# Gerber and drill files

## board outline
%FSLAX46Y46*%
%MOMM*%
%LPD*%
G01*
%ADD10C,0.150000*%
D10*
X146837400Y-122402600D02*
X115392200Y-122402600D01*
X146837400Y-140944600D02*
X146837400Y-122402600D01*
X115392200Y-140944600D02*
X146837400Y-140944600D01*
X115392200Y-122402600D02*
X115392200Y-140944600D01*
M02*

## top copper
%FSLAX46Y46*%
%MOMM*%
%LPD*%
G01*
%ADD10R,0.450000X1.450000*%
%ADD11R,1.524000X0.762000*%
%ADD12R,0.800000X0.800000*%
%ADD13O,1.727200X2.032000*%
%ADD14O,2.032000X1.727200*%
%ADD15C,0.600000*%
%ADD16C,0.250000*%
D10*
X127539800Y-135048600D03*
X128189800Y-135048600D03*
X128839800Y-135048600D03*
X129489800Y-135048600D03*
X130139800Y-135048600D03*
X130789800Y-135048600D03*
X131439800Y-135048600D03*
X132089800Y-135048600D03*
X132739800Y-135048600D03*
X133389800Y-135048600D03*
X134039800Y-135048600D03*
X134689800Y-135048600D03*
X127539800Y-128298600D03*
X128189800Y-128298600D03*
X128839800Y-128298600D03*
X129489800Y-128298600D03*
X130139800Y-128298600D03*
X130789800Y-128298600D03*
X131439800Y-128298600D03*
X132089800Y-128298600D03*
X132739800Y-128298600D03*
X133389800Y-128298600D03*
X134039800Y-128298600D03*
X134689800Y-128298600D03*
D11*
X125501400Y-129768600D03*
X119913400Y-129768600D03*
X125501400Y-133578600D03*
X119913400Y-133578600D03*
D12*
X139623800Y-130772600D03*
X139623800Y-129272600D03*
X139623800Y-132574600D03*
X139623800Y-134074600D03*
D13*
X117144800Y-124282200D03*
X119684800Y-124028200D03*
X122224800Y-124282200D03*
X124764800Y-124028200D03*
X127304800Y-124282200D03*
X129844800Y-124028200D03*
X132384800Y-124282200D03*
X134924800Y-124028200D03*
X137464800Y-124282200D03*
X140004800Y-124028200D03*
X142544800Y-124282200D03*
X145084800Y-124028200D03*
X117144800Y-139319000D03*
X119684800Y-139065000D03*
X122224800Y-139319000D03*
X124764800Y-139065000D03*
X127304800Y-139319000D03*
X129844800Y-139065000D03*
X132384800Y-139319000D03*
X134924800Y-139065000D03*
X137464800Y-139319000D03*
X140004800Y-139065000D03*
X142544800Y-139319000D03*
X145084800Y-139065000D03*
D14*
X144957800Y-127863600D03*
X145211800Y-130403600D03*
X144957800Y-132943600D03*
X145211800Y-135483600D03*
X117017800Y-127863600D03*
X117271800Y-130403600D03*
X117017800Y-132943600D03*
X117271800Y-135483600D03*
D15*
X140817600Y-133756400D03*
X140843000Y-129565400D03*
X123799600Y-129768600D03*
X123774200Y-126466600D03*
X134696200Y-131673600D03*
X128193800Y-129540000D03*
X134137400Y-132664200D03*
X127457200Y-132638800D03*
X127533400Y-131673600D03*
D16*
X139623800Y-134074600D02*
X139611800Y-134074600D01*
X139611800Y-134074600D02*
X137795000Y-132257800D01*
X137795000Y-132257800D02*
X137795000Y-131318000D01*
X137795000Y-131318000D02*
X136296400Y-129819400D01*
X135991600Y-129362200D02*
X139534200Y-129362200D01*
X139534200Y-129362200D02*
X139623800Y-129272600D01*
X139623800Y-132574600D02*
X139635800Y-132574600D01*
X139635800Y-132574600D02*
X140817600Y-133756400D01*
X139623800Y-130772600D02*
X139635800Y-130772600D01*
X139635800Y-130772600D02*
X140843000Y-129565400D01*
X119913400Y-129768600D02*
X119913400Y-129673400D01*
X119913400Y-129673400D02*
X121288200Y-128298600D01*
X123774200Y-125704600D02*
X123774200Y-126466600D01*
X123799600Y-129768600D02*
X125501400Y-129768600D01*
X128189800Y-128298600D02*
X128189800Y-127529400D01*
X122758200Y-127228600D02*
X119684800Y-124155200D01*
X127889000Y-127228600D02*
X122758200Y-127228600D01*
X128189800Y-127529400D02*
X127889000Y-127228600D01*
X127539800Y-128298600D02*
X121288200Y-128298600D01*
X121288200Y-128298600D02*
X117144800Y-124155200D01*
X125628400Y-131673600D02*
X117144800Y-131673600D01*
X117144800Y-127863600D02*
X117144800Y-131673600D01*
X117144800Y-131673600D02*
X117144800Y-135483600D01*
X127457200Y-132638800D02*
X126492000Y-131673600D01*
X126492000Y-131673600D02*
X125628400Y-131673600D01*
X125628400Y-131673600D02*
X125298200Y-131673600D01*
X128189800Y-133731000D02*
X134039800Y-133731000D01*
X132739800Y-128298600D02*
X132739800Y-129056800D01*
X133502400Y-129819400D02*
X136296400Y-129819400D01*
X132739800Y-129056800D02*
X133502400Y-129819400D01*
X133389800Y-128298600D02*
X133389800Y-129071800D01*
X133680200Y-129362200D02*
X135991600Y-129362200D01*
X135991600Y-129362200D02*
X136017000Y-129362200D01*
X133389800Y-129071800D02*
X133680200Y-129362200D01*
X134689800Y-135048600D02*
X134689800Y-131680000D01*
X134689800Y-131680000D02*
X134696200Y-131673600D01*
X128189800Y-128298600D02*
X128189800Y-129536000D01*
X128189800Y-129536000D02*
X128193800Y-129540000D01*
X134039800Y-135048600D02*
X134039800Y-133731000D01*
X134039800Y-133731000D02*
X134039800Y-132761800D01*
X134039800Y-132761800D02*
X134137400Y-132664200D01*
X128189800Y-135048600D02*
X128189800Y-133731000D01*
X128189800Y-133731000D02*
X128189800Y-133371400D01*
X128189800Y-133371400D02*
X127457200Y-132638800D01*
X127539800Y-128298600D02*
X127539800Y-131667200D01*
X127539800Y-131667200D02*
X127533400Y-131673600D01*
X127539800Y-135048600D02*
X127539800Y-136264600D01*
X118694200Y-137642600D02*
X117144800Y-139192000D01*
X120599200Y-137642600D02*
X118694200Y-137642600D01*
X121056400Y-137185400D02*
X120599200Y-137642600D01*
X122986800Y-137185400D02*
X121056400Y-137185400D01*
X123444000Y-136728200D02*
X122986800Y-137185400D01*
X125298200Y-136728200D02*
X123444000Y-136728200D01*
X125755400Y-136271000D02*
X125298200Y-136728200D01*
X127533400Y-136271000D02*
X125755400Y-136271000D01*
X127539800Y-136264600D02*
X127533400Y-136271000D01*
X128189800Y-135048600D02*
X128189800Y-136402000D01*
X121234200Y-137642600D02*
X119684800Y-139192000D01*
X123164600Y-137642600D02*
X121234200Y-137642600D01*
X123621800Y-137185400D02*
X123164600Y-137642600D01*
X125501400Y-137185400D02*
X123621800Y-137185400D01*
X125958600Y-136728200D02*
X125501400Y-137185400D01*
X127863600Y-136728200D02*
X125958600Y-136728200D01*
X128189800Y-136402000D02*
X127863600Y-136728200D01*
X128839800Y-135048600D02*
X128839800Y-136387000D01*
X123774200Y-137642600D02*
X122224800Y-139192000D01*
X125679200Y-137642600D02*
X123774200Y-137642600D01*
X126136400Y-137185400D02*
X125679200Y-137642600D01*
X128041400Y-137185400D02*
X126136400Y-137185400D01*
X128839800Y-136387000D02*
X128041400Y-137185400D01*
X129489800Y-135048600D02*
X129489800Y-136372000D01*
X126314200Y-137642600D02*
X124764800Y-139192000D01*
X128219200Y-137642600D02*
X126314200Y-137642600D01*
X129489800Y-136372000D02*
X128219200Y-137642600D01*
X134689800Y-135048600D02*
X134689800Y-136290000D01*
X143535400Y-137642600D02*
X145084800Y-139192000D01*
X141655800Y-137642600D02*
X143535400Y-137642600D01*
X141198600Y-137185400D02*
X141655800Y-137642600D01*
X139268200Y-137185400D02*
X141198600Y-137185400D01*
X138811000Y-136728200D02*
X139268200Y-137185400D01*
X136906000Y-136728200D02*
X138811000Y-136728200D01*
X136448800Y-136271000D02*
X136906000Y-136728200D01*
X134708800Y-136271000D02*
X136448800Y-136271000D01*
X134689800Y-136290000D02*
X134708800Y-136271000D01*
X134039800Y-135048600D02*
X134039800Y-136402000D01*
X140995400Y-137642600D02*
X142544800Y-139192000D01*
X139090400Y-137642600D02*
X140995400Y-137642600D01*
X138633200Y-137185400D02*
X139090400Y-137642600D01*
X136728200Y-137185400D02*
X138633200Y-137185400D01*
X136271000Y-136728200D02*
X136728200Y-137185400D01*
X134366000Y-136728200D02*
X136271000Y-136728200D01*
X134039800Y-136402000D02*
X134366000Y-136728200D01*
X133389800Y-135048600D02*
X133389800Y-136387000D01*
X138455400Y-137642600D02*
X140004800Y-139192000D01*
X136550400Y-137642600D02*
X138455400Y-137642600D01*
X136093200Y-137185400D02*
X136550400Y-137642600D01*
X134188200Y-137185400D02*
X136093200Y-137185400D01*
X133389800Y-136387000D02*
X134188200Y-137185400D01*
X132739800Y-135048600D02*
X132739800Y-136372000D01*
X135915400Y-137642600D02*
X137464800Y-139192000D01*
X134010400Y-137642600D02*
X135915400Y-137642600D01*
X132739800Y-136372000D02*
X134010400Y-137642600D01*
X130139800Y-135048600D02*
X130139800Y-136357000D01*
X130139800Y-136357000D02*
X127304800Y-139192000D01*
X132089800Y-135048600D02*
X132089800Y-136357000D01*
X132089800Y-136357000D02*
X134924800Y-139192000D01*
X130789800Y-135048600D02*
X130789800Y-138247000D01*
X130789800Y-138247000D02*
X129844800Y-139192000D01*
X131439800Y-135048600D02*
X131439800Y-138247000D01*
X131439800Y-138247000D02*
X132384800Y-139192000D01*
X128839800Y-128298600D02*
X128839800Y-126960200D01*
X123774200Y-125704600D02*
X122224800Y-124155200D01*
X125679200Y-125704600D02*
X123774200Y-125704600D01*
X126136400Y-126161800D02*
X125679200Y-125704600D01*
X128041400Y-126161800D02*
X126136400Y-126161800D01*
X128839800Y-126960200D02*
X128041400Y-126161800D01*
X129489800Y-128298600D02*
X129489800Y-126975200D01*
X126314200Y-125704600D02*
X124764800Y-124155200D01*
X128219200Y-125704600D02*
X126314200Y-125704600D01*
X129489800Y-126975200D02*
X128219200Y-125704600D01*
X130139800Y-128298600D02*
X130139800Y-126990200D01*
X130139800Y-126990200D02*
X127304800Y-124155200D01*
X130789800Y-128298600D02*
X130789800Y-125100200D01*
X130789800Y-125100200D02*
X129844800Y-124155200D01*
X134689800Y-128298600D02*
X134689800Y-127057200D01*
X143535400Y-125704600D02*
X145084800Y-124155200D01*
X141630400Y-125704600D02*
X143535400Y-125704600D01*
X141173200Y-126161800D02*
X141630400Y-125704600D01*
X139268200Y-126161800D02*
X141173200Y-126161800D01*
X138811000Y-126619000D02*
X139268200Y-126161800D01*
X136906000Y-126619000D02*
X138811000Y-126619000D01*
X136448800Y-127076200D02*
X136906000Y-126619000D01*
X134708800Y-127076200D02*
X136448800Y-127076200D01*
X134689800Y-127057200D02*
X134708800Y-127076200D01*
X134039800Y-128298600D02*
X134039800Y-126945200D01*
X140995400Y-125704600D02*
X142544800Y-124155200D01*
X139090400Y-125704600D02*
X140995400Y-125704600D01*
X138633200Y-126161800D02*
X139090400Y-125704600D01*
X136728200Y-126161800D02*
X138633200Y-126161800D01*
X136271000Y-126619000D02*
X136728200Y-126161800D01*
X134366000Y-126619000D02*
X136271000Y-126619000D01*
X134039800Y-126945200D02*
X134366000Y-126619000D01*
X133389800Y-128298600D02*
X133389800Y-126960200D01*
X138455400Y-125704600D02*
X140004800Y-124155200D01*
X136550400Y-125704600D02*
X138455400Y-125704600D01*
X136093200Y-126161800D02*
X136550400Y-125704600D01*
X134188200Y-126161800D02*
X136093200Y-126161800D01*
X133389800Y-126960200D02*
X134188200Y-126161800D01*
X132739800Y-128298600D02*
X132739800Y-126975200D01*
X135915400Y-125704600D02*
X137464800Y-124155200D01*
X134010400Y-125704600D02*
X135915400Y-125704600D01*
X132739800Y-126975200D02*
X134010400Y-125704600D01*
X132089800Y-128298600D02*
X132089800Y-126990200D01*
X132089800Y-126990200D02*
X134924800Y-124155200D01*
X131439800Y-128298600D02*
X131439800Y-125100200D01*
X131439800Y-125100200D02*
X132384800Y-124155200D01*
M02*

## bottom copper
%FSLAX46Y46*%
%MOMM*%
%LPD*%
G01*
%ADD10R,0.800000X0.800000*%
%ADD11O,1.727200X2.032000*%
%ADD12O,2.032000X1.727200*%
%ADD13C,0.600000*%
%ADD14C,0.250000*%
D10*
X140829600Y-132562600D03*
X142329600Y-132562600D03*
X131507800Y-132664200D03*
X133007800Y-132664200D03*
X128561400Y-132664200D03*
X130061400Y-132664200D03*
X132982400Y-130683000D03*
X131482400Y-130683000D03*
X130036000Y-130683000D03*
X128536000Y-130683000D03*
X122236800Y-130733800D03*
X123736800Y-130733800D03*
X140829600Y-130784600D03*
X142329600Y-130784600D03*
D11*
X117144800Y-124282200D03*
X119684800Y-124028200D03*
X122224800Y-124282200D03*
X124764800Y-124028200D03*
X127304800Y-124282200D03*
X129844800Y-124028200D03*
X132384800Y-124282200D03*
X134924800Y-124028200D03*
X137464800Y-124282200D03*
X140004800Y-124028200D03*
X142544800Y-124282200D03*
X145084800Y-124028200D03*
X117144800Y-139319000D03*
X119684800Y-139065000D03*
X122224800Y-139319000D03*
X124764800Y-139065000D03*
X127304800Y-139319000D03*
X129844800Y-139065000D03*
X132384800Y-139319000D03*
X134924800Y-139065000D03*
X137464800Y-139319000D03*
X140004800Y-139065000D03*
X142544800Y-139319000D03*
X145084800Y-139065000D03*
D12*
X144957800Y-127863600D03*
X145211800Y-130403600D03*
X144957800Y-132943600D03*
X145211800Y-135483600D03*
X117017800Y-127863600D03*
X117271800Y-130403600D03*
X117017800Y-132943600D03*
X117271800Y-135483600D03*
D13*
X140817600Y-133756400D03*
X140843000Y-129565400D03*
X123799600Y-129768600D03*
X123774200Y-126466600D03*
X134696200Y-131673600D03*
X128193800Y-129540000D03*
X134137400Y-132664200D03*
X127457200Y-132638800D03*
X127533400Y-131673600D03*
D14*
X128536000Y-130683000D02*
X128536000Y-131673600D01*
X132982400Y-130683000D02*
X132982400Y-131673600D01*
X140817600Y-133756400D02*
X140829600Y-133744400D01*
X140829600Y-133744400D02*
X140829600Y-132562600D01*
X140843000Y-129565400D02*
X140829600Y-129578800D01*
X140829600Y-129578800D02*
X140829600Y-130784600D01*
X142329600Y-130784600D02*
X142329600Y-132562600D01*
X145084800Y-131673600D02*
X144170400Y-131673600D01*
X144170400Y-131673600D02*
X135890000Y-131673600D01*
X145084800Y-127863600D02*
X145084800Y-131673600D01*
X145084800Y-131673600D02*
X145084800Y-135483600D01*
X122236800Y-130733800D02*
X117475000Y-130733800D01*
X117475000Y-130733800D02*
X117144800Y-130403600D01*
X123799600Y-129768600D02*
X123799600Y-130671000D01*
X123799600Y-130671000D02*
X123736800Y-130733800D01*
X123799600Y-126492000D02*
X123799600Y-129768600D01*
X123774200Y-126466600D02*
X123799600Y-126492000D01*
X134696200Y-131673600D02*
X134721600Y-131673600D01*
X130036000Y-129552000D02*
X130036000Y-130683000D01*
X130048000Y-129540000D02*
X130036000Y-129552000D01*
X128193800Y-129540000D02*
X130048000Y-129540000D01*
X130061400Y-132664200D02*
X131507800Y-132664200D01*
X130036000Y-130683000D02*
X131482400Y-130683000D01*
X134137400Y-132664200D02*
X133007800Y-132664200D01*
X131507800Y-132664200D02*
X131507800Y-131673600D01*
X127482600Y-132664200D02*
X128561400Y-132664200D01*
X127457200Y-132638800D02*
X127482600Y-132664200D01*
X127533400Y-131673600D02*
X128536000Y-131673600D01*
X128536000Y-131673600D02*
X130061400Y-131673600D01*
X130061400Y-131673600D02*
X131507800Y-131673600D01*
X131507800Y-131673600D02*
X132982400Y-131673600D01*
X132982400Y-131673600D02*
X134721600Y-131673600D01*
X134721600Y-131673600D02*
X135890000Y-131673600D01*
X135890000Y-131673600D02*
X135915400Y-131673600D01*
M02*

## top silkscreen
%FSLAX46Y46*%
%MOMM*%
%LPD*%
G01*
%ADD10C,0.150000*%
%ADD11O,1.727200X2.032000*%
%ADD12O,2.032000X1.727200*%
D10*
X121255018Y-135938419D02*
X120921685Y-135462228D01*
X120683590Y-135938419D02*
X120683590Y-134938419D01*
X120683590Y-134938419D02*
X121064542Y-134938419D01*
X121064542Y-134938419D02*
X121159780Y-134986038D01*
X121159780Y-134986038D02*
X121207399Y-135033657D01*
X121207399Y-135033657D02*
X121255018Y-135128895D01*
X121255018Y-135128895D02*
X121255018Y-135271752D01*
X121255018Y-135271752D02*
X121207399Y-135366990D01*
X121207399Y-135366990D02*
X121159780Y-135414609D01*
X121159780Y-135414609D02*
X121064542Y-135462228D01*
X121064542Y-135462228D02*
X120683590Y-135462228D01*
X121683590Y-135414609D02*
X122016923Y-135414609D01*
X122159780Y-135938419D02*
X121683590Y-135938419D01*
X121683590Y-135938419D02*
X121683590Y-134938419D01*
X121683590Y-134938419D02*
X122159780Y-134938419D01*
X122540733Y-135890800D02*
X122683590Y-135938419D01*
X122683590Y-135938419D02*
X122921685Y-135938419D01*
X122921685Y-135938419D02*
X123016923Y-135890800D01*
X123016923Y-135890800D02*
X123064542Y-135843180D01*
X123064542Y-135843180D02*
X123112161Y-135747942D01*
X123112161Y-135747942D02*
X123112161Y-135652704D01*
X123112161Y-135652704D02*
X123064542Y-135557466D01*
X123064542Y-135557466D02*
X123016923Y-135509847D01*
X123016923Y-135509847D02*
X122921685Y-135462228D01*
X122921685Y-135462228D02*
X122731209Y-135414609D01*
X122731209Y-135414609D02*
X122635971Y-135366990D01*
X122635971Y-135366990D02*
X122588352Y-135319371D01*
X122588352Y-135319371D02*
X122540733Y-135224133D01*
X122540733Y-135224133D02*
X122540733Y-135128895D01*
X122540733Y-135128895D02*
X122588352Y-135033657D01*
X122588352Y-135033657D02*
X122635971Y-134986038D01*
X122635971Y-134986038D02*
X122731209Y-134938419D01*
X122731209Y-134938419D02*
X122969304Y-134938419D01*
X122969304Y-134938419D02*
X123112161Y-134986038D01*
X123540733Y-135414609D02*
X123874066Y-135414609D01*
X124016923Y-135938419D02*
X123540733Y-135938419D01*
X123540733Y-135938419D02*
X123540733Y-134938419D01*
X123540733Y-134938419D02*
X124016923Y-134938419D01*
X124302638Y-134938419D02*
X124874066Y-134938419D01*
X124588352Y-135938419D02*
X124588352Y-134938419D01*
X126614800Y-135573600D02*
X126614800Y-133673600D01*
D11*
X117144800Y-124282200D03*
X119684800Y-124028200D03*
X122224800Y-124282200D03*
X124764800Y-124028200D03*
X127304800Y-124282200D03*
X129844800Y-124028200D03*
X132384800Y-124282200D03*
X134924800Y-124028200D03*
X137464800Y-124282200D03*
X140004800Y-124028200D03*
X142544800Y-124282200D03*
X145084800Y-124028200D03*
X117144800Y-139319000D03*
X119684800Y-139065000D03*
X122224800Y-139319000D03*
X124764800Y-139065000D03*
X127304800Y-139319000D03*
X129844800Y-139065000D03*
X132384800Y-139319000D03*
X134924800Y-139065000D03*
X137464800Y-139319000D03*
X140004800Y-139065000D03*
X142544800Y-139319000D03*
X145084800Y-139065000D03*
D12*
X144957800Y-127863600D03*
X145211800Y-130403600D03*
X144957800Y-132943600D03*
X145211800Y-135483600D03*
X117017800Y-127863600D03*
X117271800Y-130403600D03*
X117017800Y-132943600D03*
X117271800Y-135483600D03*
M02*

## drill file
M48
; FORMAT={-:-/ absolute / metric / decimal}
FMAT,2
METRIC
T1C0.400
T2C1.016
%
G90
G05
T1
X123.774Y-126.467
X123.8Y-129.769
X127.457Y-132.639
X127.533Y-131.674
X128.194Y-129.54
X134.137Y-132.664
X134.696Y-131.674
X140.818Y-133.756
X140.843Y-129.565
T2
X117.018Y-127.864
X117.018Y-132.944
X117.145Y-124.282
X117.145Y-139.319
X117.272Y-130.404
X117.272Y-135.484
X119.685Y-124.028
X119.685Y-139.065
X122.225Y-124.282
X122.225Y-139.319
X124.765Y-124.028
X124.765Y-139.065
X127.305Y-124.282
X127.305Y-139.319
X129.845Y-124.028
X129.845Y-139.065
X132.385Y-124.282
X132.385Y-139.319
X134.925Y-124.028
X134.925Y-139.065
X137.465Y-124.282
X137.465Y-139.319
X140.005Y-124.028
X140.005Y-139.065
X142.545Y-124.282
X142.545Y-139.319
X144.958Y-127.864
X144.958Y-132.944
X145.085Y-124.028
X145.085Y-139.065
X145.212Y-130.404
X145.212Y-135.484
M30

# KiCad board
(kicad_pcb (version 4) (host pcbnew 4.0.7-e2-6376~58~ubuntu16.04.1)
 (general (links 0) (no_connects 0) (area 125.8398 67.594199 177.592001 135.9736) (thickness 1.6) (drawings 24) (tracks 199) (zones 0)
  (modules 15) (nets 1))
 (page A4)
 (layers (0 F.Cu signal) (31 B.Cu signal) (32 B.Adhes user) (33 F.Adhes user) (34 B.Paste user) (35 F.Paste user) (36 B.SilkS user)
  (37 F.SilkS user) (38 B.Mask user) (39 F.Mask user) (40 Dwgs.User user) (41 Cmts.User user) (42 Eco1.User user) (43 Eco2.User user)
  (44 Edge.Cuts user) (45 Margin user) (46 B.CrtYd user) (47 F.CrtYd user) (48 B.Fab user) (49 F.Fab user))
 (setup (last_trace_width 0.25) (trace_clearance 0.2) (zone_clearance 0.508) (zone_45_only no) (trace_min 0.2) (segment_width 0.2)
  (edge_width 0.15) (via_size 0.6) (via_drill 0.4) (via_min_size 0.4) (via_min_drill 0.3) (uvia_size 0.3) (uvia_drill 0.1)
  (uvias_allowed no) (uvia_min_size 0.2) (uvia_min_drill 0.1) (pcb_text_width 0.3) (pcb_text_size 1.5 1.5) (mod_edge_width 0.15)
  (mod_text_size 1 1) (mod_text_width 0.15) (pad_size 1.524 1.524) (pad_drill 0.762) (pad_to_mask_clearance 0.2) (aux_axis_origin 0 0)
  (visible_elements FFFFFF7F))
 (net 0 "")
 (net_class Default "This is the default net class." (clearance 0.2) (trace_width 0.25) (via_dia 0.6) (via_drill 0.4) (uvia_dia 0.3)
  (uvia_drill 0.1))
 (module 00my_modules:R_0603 (layer B.Cu) (at 141.5796 132.5626)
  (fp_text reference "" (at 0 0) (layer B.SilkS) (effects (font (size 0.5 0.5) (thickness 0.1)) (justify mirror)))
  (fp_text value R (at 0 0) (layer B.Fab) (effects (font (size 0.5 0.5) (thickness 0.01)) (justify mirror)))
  (pad 1 smd rect (at -0.75 0) (size 0.8 0.8) (layers B.Cu B.Paste B.Mask))
  (pad 2 smd rect (at 0.75 0) (size 0.8 0.8) (layers B.Cu B.Paste B.Mask)))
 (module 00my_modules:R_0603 (layer B.Cu) (at 132.2578 132.6642)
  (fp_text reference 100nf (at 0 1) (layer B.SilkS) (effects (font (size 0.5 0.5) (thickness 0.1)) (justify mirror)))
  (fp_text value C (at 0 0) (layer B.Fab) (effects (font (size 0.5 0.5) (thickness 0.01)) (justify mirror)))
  (pad 1 smd rect (at -0.75 0) (size 0.8 0.8) (layers B.Cu B.Paste B.Mask))
  (pad 2 smd rect (at 0.75 0) (size 0.8 0.8) (layers B.Cu B.Paste B.Mask)))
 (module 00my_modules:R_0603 (layer B.Cu) (at 129.3114 132.6642)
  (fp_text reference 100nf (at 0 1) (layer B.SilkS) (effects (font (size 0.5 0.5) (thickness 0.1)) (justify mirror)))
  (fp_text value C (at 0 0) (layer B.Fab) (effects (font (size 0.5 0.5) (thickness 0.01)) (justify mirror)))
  (pad 1 smd rect (at -0.75 0) (size 0.8 0.8) (layers B.Cu B.Paste B.Mask))
  (pad 2 smd rect (at 0.75 0) (size 0.8 0.8) (layers B.Cu B.Paste B.Mask)))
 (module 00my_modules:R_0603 (layer B.Cu) (at 132.2324 130.683 180)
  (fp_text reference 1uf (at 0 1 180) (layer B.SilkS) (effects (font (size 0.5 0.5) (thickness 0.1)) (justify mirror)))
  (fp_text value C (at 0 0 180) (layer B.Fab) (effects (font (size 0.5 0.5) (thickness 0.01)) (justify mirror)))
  (pad 1 smd rect (at -0.75 0 180) (size 0.8 0.8) (layers B.Cu B.Paste B.Mask))
  (pad 2 smd rect (at 0.75 0 180) (size 0.8 0.8) (layers B.Cu B.Paste B.Mask)))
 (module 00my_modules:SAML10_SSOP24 (layer F.Cu) (at 131.1148 131.6736 90)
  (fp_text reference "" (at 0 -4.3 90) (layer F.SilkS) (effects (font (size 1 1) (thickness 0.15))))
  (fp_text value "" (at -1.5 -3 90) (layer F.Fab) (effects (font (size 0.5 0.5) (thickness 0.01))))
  (fp_line (start -3.9 -4.5) (end -2 -4.5) (layer F.SilkS) (width 0.15))
  (pad VOUT smd rect (at -3.375 -3.575 90) (size 1.45 0.45) (layers F.Cu F.Paste F.Mask))
  (pad VIO smd rect (at -3.375 -2.925 90) (size 1.45 0.45) (layers F.Cu F.Paste F.Mask))
  (pad SWCL smd rect (at -3.375 -2.275 90) (size 1.45 0.45) (layers F.Cu F.Paste F.Mask))
  (pad SWDI smd rect (at -3.375 -1.625 90) (size 1.45 0.45) (layers F.Cu F.Paste F.Mask))
  (pad PA00 smd rect (at -3.375 -0.975 90) (size 1.45 0.45) (layers F.Cu F.Paste F.Mask))
  (pad PA01 smd rect (at -3.375 -0.325 90) (size 1.45 0.45) (layers F.Cu F.Paste F.Mask))
  (pad PA02 smd rect (at -3.375 0.325 90) (size 1.45 0.45) (layers F.Cu F.Paste F.Mask))
  (pad PA03 smd rect (at -3.375 0.975 90) (size 1.45 0.45) (layers F.Cu F.Paste F.Mask))
  (pad PA04 smd rect (at -3.375 1.625 90) (size 1.45 0.45) (layers F.Cu F.Paste F.Mask))
  (pad PA05 smd rect (at -3.375 2.275 90) (size 1.45 0.45) (layers F.Cu F.Paste F.Mask))
  (pad VANA smd rect (at -3.375 2.925 90) (size 1.45 0.45) (layers F.Cu F.Paste F.Mask))
  (pad GANA smd rect (at -3.375 3.575 90) (size 1.45 0.45) (layers F.Cu F.Paste F.Mask))
  (pad GND smd rect (at 3.375 -3.575 90) (size 1.45 0.45) (layers F.Cu F.Paste F.Mask))
  (pad VCOR smd rect (at 3.375 -2.925 90) (size 1.45 0.45) (layers F.Cu F.Paste F.Mask))
  (pad RSTN smd rect (at 3.375 -2.275 90) (size 1.45 0.45) (layers F.Cu F.Paste F.Mask))
  (pad PA23 smd rect (at 3.375 -1.625 90) (size 1.45 0.45) (layers F.Cu F.Paste F.Mask))
  (pad PA22 smd rect (at 3.375 -0.975 90) (size 1.45 0.45) (layers F.Cu F.Paste F.Mask))
  (pad PA19 smd rect (at 3.375 -0.325 90) (size 1.45 0.45) (layers F.Cu F.Paste F.Mask))
  (pad PA18 smd rect (at 3.375 0.325 90) (size 1.45 0.45) (layers F.Cu F.Paste F.Mask))
  (pad PA17 smd rect (at 3.375 0.975 90) (size 1.45 0.45) (layers F.Cu F.Paste F.Mask))
  (pad PA16 smd rect (at 3.375 1.625 90) (size 1.45 0.45) (layers F.Cu F.Paste F.Mask))
  (pad PA15 smd rect (at 3.375 2.275 90) (size 1.45 0.45) (layers F.Cu F.Paste F.Mask))
  (pad PA14 smd rect (at 3.375 2.925 90) (size 1.45 0.45) (layers F.Cu F.Paste F.Mask))
  (pad PA08 smd rect (at 3.375 3.575 90) (size 1.45 0.45) (layers F.Cu F.Paste F.Mask)))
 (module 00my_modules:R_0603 (layer B.Cu) (at 129.286 130.683 180)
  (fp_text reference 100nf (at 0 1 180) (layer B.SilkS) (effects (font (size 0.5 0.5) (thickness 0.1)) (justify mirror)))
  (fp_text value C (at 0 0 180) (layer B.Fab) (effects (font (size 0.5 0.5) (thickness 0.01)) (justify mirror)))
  (pad 1 smd rect (at -0.75 0 180) (size 0.8 0.8) (layers B.Cu B.Paste B.Mask))
  (pad 2 smd rect (at 0.75 0 180) (size 0.8 0.8) (layers B.Cu B.Paste B.Mask)))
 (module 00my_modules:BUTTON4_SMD (layer F.Cu) (at 122.7074 131.6736 180)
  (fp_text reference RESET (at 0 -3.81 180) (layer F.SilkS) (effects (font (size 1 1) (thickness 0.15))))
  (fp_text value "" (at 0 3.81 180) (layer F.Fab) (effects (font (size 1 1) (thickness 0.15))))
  (pad 1 smd rect (at -2.794 1.905 180) (size 1.524 0.762) (layers F.Cu F.Paste F.Mask))
  (pad 2 smd rect (at 2.794 1.905 180) (size 1.524 0.762) (layers F.Cu F.Paste F.Mask))
  (pad 3 smd rect (at -2.794 -1.905 180) (size 1.524 0.762) (layers F.Cu F.Paste F.Mask))
  (pad 4 smd rect (at 2.794 -1.905 180) (size 1.524 0.762) (layers F.Cu F.Paste F.Mask)))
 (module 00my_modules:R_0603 (layer B.Cu) (at 122.9868 130.7338)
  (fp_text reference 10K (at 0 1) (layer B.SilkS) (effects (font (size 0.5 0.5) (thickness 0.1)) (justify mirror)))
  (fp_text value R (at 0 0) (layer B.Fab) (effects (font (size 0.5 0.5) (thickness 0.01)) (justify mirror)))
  (pad 1 smd rect (at -0.75 0) (size 0.8 0.8) (layers B.Cu B.Paste B.Mask))
  (pad 2 smd rect (at 0.75 0) (size 0.8 0.8) (layers B.Cu B.Paste B.Mask)))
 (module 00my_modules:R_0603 (layer B.Cu) (at 141.5796 130.7846)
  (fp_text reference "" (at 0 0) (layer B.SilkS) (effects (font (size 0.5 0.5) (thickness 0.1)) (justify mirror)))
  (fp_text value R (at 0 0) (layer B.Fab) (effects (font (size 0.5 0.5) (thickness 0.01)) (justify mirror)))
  (pad 1 smd rect (at -0.75 0) (size 0.8 0.8) (layers B.Cu B.Paste B.Mask))
  (pad 2 smd rect (at 0.75 0) (size 0.8 0.8) (layers B.Cu B.Paste B.Mask)))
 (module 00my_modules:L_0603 (layer F.Cu) (at 139.6238 130.0226 90)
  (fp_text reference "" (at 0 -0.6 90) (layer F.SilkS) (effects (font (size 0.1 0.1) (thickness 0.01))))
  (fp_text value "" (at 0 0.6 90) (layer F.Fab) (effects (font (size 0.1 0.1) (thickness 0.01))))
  (pad 1 smd rect (at -0.75 0 90) (size 0.8 0.8) (layers F.Cu F.Paste F.Mask))
  (pad 2 smd rect (at 0.75 0 90) (size 0.8 0.8) (layers F.Cu F.Paste F.Mask)))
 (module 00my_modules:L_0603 (layer F.Cu) (at 139.6238 133.3246 270)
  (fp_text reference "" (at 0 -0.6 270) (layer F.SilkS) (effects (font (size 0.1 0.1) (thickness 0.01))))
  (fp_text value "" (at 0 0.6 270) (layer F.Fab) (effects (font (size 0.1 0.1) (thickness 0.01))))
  (pad 1 smd rect (at -0.75 0 270) (size 0.8 0.8) (layers F.Cu F.Paste F.Mask))
  (pad 2 smd rect (at 0.75 0 270) (size 0.8 0.8) (layers F.Cu F.Paste F.Mask)))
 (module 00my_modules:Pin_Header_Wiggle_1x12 (layer F.Cu) (at 117.1448 124.1552 90)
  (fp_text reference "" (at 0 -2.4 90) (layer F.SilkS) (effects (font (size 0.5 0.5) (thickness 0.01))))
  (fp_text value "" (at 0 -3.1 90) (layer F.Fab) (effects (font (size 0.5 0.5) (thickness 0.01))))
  (pad 1 thru_hole oval (at -0.127 0 90) (size 2.032 1.7272) (drill 1.016) (layers *.Cu *.Mask F.SilkS))
  (pad 2 thru_hole oval (at 0.127 2.54 90) (size 2.032 1.7272) (drill 1.016) (layers *.Cu *.Mask F.SilkS))
  (pad 3 thru_hole oval (at -0.127 5.08 90) (size 2.032 1.7272) (drill 1.016) (layers *.Cu *.Mask F.SilkS))
  (pad 4 thru_hole oval (at 0.127 7.62 90) (size 2.032 1.7272) (drill 1.016) (layers *.Cu *.Mask F.SilkS))
  (pad 5 thru_hole oval (at -0.127 10.16 90) (size 2.032 1.7272) (drill 1.016) (layers *.Cu *.Mask F.SilkS))
  (pad 6 thru_hole oval (at 0.127 12.7 90) (size 2.032 1.7272) (drill 1.016) (layers *.Cu *.Mask F.SilkS))
  (pad 7 thru_hole oval (at -0.127 15.24 90) (size 2.032 1.7272) (drill 1.016) (layers *.Cu *.Mask F.SilkS))
  (pad 8 thru_hole oval (at 0.127 17.78 90) (size 2.032 1.7272) (drill 1.016) (layers *.Cu *.Mask F.SilkS))
  (pad 9 thru_hole oval (at -0.127 20.32 90) (size 2.032 1.7272) (drill 1.016) (layers *.Cu *.Mask F.SilkS))
  (pad 10 thru_hole oval (at 0.127 22.86 90) (size 2.032 1.7272) (drill 1.016) (layers *.Cu *.Mask F.SilkS))
  (pad 11 thru_hole oval (at -0.127 25.4 90) (size 2.032 1.7272) (drill 1.016) (layers *.Cu *.Mask F.SilkS))
  (pad 12 thru_hole oval (at 0.127 27.94 90) (size 2.032 1.7272) (drill 1.016) (layers *.Cu *.Mask F.SilkS)))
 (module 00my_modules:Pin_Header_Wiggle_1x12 (layer F.Cu) (at 117.1448 139.192 90)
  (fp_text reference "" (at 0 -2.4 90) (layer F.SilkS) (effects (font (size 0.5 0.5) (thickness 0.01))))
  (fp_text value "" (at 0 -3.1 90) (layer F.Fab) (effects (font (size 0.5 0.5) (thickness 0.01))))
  (pad 1 thru_hole oval (at -0.127 0 90) (size 2.032 1.7272) (drill 1.016) (layers *.Cu *.Mask F.SilkS))
  (pad 2 thru_hole oval (at 0.127 2.54 90) (size 2.032 1.7272) (drill 1.016) (layers *.Cu *.Mask F.SilkS))
  (pad 3 thru_hole oval (at -0.127 5.08 90) (size 2.032 1.7272) (drill 1.016) (layers *.Cu *.Mask F.SilkS))
  (pad 4 thru_hole oval (at 0.127 7.62 90) (size 2.032 1.7272) (drill 1.016) (layers *.Cu *.Mask F.SilkS))
  (pad 5 thru_hole oval (at -0.127 10.16 90) (size 2.032 1.7272) (drill 1.016) (layers *.Cu *.Mask F.SilkS))
  (pad 6 thru_hole oval (at 0.127 12.7 90) (size 2.032 1.7272) (drill 1.016) (layers *.Cu *.Mask F.SilkS))
  (pad 7 thru_hole oval (at -0.127 15.24 90) (size 2.032 1.7272) (drill 1.016) (layers *.Cu *.Mask F.SilkS))
  (pad 8 thru_hole oval (at 0.127 17.78 90) (size 2.032 1.7272) (drill 1.016) (layers *.Cu *.Mask F.SilkS))
  (pad 9 thru_hole oval (at -0.127 20.32 90) (size 2.032 1.7272) (drill 1.016) (layers *.Cu *.Mask F.SilkS))
  (pad 10 thru_hole oval (at 0.127 22.86 90) (size 2.032 1.7272) (drill 1.016) (layers *.Cu *.Mask F.SilkS))
  (pad 11 thru_hole oval (at -0.127 25.4 90) (size 2.032 1.7272) (drill 1.016) (layers *.Cu *.Mask F.SilkS))
  (pad 12 thru_hole oval (at 0.127 27.94 90) (size 2.032 1.7272) (drill 1.016) (layers *.Cu *.Mask F.SilkS)))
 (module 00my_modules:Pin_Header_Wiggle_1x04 (layer F.Cu) (at 145.0848 127.8636)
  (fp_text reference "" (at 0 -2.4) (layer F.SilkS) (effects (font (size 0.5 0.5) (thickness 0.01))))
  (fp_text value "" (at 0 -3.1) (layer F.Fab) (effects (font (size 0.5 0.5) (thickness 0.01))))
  (pad 1 thru_hole oval (at -0.127 0) (size 2.032 1.7272) (drill 1.016) (layers *.Cu *.Mask F.SilkS))
  (pad 2 thru_hole oval (at 0.127 2.54) (size 2.032 1.7272) (drill 1.016) (layers *.Cu *.Mask F.SilkS))
  (pad 3 thru_hole oval (at -0.127 5.08) (size 2.032 1.7272) (drill 1.016) (layers *.Cu *.Mask F.SilkS))
  (pad 4 thru_hole oval (at 0.127 7.62) (size 2.032 1.7272) (drill 1.016) (layers *.Cu *.Mask F.SilkS)))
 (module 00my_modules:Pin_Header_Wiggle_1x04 (layer F.Cu) (at 117.1448 127.8636)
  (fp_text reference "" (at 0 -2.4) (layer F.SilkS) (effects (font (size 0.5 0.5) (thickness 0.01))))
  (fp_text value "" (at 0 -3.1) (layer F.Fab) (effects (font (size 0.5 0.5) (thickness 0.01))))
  (pad 1 thru_hole oval (at -0.127 0) (size 2.032 1.7272) (drill 1.016) (layers *.Cu *.Mask F.SilkS))
  (pad 2 thru_hole oval (at 0.127 2.54) (size 2.032 1.7272) (drill 1.016) (layers *.Cu *.Mask F.SilkS))
  (pad 3 thru_hole oval (at -0.127 5.08) (size 2.032 1.7272) (drill 1.016) (layers *.Cu *.Mask F.SilkS))
  (pad 4 thru_hole oval (at 0.127 7.62) (size 2.032 1.7272) (drill 1.016) (layers *.Cu *.Mask F.SilkS)))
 (gr_line (start 146.8374 122.4026) (end 115.3922 122.4026) (angle 90) (layer Edge.Cuts) (width 0.15))
 (gr_line (start 146.8374 140.9446) (end 146.8374 122.4026) (angle 90) (layer Edge.Cuts) (width 0.15))
 (gr_line (start 115.3922 140.9446) (end 146.8374 140.9446) (angle 90) (layer Edge.Cuts) (width 0.15))
 (gr_line (start 115.3922 122.4026) (end 115.3922 140.9446) (angle 90) (layer Edge.Cuts) (width 0.15))
 (segment (start 128.536 130.683) (end 128.536 131.6736) (width 0.25) (layer B.Cu) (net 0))
 (segment (start 132.9824 130.683) (end 132.9824 131.6736) (width 0.25) (layer B.Cu) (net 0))
 (segment (start 139.6238 134.0746) (end 139.6118 134.0746) (width 0.25) (layer F.Cu) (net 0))
 (segment (start 139.6118 134.0746) (end 137.795 132.2578) (width 0.25) (layer F.Cu) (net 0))
 (segment (start 137.795 132.2578) (end 137.795 131.318) (width 0.25) (layer F.Cu) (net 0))
 (segment (start 137.795 131.318) (end 136.2964 129.8194) (width 0.25) (layer F.Cu) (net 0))
 (segment (start 135.9916 129.3622) (end 139.5342 129.3622) (width 0.25) (layer F.Cu) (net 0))
 (segment (start 139.5342 129.3622) (end 139.6238 129.2726) (width 0.25) (layer F.Cu) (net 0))
 (segment (start 139.6238 132.5746) (end 139.6358 132.5746) (width 0.25) (layer F.Cu) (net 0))
 (segment (start 139.6358 132.5746) (end 140.8176 133.7564) (width 0.25) (layer F.Cu) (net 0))
 (via (at 140.8176 133.7564) (size 0.6) (drill 0.4) (layers F.Cu B.Cu) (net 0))
 (segment (start 140.8176 133.7564) (end 140.8296 133.7444) (width 0.25) (layer B.Cu) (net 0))
 (segment (start 140.8296 133.7444) (end 140.8296 132.5626) (width 0.25) (layer B.Cu) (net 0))
 (segment (start 139.6238 130.7726) (end 139.6358 130.7726) (width 0.25) (layer F.Cu) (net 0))
 (segment (start 139.6358 130.7726) (end 140.843 129.5654) (width 0.25) (layer F.Cu) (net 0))
 (via (at 140.843 129.5654) (size 0.6) (drill 0.4) (layers F.Cu B.Cu) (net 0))
 (segment (start 140.843 129.5654) (end 140.8296 129.5788) (width 0.25) (layer B.Cu) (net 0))
 (segment (start 140.8296 129.5788) (end 140.8296 130.7846) (width 0.25) (layer B.Cu) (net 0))
 (segment (start 142.3296 130.7846) (end 142.3296 132.5626) (width 0.25) (layer B.Cu) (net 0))
 (segment (start 145.0848 131.6736) (end 144.1704 131.6736) (width 0.25) (layer B.Cu) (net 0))
 (segment (start 144.1704 131.6736) (end 135.89 131.6736) (width 0.25) (layer B.Cu) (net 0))
 (segment (start 145.0848 127.8636) (end 145.0848 131.6736) (width 0.25) (layer B.Cu) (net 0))
 (segment (start 145.0848 131.6736) (end 145.0848 135.4836) (width 0.25) (layer B.Cu) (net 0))
 (segment (start 122.2368 130.7338) (end 117.475 130.7338) (width 0.25) (layer B.Cu) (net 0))
 (segment (start 117.475 130.7338) (end 117.1448 130.4036) (width 0.25) (layer B.Cu) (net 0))
 (segment (start 123.7996 129.7686) (end 123.7996 130.671) (width 0.25) (layer B.Cu) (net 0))
 (segment (start 123.7996 130.671) (end 123.7368 130.7338) (width 0.25) (layer B.Cu) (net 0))
 (segment (start 119.9134 129.7686) (end 119.9134 129.6734) (width 0.25) (layer F.Cu) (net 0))
 (segment (start 119.9134 129.6734) (end 121.2882 128.2986) (width 0.25) (layer F.Cu) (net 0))
 (segment (start 123.7742 125.7046) (end 123.7742 126.4666) (width 0.25) (layer F.Cu) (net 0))
 (segment (start 123.7996 129.7686) (end 125.5014 129.7686) (width 0.25) (layer F.Cu) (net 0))
 (via (at 123.7996 129.7686) (size 0.6) (drill 0.4) (layers F.Cu B.Cu) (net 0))
 (segment (start 123.7996 126.492) (end 123.7996 129.7686) (width 0.25) (layer B.Cu) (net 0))
 (segment (start 123.7742 126.4666) (end 123.7996 126.492) (width 0.25) (layer B.Cu) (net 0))
 (via (at 123.7742 126.4666) (size 0.6) (drill 0.4) (layers F.Cu B.Cu) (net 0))
 (segment (start 128.1898 128.2986) (end 128.1898 127.5294) (width 0.25) (layer F.Cu) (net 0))
 (segment (start 122.7582 127.2286) (end 119.6848 124.1552) (width 0.25) (layer F.Cu) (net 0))
 (segment (start 127.889 127.2286) (end 122.7582 127.2286) (width 0.25) (layer F.Cu) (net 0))
 (segment (start 128.1898 127.5294) (end 127.889 127.2286) (width 0.25) (layer F.Cu) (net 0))
 (segment (start 127.5398 128.2986) (end 121.2882 128.2986) (width 0.25) (layer F.Cu) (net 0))
 (segment (start 121.2882 128.2986) (end 117.1448 124.1552) (width 0.25) (layer F.Cu) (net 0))
 (segment (start 125.6284 131.6736) (end 117.1448 131.6736) (width 0.25) (layer F.Cu) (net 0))
 (segment (start 117.1448 127.8636) (end 117.1448 131.6736) (width 0.25) (layer F.Cu) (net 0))
 (segment (start 117.1448 131.6736) (end 117.1448 135.4836) (width 0.25) (layer F.Cu) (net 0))
 (segment (start 127.4572 132.6388) (end 126.492 131.6736) (width 0.25) (layer F.Cu) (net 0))
 (segment (start 126.492 131.6736) (end 125.6284 131.6736) (width 0.25) (layer F.Cu) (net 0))
 (segment (start 125.6284 131.6736) (end 125.2982 131.6736) (width 0.25) (layer F.Cu) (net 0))
 (segment (start 128.1898 133.731) (end 134.0398 133.731) (width 0.25) (layer F.Cu) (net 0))
 (segment (start 132.7398 128.2986) (end 132.7398 129.0568) (width 0.25) (layer F.Cu) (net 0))
 (segment (start 133.5024 129.8194) (end 136.2964 129.8194) (width 0.25) (layer F.Cu) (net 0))
 (segment (start 132.7398 129.0568) (end 133.5024 129.8194) (width 0.25) (layer F.Cu) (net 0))
 (segment (start 133.3898 128.2986) (end 133.3898 129.0718) (width 0.25) (layer F.Cu) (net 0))
 (segment (start 133.6802 129.3622) (end 135.9916 129.3622) (width 0.25) (layer F.Cu) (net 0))
 (segment (start 135.9916 129.3622) (end 136.017 129.3622) (width 0.25) (layer F.Cu) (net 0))
 (segment (start 133.3898 129.0718) (end 133.6802 129.3622) (width 0.25) (layer F.Cu) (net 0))
 (segment (start 134.6898 135.0486) (end 134.6898 131.68) (width 0.25) (layer F.Cu) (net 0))
 (segment (start 134.6962 131.6736) (end 134.7216 131.6736) (width 0.25) (layer B.Cu) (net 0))
 (via (at 134.6962 131.6736) (size 0.6) (drill 0.4) (layers F.Cu B.Cu) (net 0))
 (segment (start 134.6898 131.68) (end 134.6962 131.6736) (width 0.25) (layer F.Cu) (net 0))
 (segment (start 128.1898 128.2986) (end 128.1898 129.536) (width 0.25) (layer F.Cu) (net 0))
 (segment (start 130.036 129.552) (end 130.036 130.683) (width 0.25) (layer B.Cu) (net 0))
 (segment (start 130.048 129.54) (end 130.036 129.552) (width 0.25) (layer B.Cu) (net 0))
 (segment (start 128.1938 129.54) (end 130.048 129.54) (width 0.25) (layer B.Cu) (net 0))
 (via (at 128.1938 129.54) (size 0.6) (drill 0.4) (layers F.Cu B.Cu) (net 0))
 (segment (start 128.1898 129.536) (end 128.1938 129.54) (width 0.25) (layer F.Cu) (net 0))
 (segment (start 130.0614 132.6642) (end 131.5078 132.6642) (width 0.25) (layer B.Cu) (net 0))
 (segment (start 130.036 130.683) (end 131.4824 130.683) (width 0.25) (layer B.Cu) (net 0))
 (segment (start 134.0398 135.0486) (end 134.0398 133.731) (width 0.25) (layer F.Cu) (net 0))
 (segment (start 134.0398 133.731) (end 134.0398 132.7618) (width 0.25) (layer F.Cu) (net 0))
 (segment (start 134.0398 132.7618) (end 134.1374 132.6642) (width 0.25) (layer F.Cu) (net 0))
 (via (at 134.1374 132.6642) (size 0.6) (drill 0.4) (layers F.Cu B.Cu) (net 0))
 (segment (start 134.1374 132.6642) (end 133.0078 132.6642) (width 0.25) (layer B.Cu) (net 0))
 (segment (start 131.5078 132.6642) (end 131.5078 131.6736) (width 0.25) (layer B.Cu) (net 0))
 (segment (start 128.1898 135.0486) (end 128.1898 133.731) (width 0.25) (layer F.Cu) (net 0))
 (segment (start 128.1898 133.731) (end 128.1898 133.3714) (width 0.25) (layer F.Cu) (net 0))
 (segment (start 127.4826 132.6642) (end 128.5614 132.6642) (width 0.25) (layer B.Cu) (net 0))
 (segment (start 127.4572 132.6388) (end 127.4826 132.6642) (width 0.25) (layer B.Cu) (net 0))
 (via (at 127.4572 132.6388) (size 0.6) (drill 0.4) (layers F.Cu B.Cu) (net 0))
 (segment (start 128.1898 133.3714) (end 127.4572 132.6388) (width 0.25) (layer F.Cu) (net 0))
 (segment (start 127.5398 128.2986) (end 127.5398 131.6672) (width 0.25) (layer F.Cu) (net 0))
 (segment (start 127.5334 131.6736) (end 128.536 131.6736) (width 0.25) (layer B.Cu) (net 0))
 (segment (start 128.536 131.6736) (end 130.0614 131.6736) (width 0.25) (layer B.Cu) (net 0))
 (segment (start 130.0614 131.6736) (end 131.5078 131.6736) (width 0.25) (layer B.Cu) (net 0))
 (segment (start 131.5078 131.6736) (end 132.9824 131.6736) (width 0.25) (layer B.Cu) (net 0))
 (segment (start 132.9824 131.6736) (end 134.7216 131.6736) (width 0.25) (layer B.Cu) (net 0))
 (segment (start 134.7216 131.6736) (end 135.89 131.6736) (width 0.25) (layer B.Cu) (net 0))
 (segment (start 135.89 131.6736) (end 135.9154 131.6736) (width 0.25) (layer B.Cu) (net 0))
 (via (at 127.5334 131.6736) (size 0.6) (drill 0.4) (layers F.Cu B.Cu) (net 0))
 (segment (start 127.5398 131.6672) (end 127.5334 131.6736) (width 0.25) (layer F.Cu) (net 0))
 (segment (start 127.5398 135.0486) (end 127.5398 136.2646) (width 0.25) (layer F.Cu) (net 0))
 (segment (start 118.6942 137.6426) (end 117.1448 139.192) (width 0.25) (layer F.Cu) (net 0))
 (segment (start 120.5992 137.6426) (end 118.6942 137.6426) (width 0.25) (layer F.Cu) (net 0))
 (segment (start 121.0564 137.1854) (end 120.5992 137.6426) (width 0.25) (layer F.Cu) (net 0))
 (segment (start 122.9868 137.1854) (end 121.0564 137.1854) (width 0.25) (layer F.Cu) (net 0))
 (segment (start 123.444 136.7282) (end 122.9868 137.1854) (width 0.25) (layer F.Cu) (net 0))
 (segment (start 125.2982 136.7282) (end 123.444 136.7282) (width 0.25) (layer F.Cu) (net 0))
 (segment (start 125.7554 136.271) (end 125.2982 136.7282) (width 0.25) (layer F.Cu) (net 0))
 (segment (start 127.5334 136.271) (end 125.7554 136.271) (width 0.25) (layer F.Cu) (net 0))
 (segment (start 127.5398 136.2646) (end 127.5334 136.271) (width 0.25) (layer F.Cu) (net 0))
 (segment (start 128.1898 135.0486) (end 128.1898 136.402) (width 0.25) (layer F.Cu) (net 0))
 (segment (start 121.2342 137.6426) (end 119.6848 139.192) (width 0.25) (layer F.Cu) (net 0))
 (segment (start 123.1646 137.6426) (end 121.2342 137.6426) (width 0.25) (layer F.Cu) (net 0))
 (segment (start 123.6218 137.1854) (end 123.1646 137.6426) (width 0.25) (layer F.Cu) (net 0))
 (segment (start 125.5014 137.1854) (end 123.6218 137.1854) (width 0.25) (layer F.Cu) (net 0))
 (segment (start 125.9586 136.7282) (end 125.5014 137.1854) (width 0.25) (layer F.Cu) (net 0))
 (segment (start 127.8636 136.7282) (end 125.9586 136.7282) (width 0.25) (layer F.Cu) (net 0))
 (segment (start 128.1898 136.402) (end 127.8636 136.7282) (width 0.25) (layer F.Cu) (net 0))
 (segment (start 128.8398 135.0486) (end 128.8398 136.387) (width 0.25) (layer F.Cu) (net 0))
 (segment (start 123.7742 137.6426) (end 122.2248 139.192) (width 0.25) (layer F.Cu) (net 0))
 (segment (start 125.6792 137.6426) (end 123.7742 137.6426) (width 0.25) (layer F.Cu) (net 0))
 (segment (start 126.1364 137.1854) (end 125.6792 137.6426) (width 0.25) (layer F.Cu) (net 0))
 (segment (start 128.0414 137.1854) (end 126.1364 137.1854) (width 0.25) (layer F.Cu) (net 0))
 (segment (start 128.8398 136.387) (end 128.0414 137.1854) (width 0.25) (layer F.Cu) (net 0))
 (segment (start 129.4898 135.0486) (end 129.4898 136.372) (width 0.25) (layer F.Cu) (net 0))
 (segment (start 126.3142 137.6426) (end 124.7648 139.192) (width 0.25) (layer F.Cu) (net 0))
 (segment (start 128.2192 137.6426) (end 126.3142 137.6426) (width 0.25) (layer F.Cu) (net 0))
 (segment (start 129.4898 136.372) (end 128.2192 137.6426) (width 0.25) (layer F.Cu) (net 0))
 (segment (start 134.6898 135.0486) (end 134.6898 136.29) (width 0.25) (layer F.Cu) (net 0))
 (segment (start 143.5354 137.6426) (end 145.0848 139.192) (width 0.25) (layer F.Cu) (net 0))
 (segment (start 141.6558 137.6426) (end 143.5354 137.6426) (width 0.25) (layer F.Cu) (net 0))
 (segment (start 141.1986 137.1854) (end 141.6558 137.6426) (width 0.25) (layer F.Cu) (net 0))
 (segment (start 139.2682 137.1854) (end 141.1986 137.1854) (width 0.25) (layer F.Cu) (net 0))
 (segment (start 138.811 136.7282) (end 139.2682 137.1854) (width 0.25) (layer F.Cu) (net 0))
 (segment (start 136.906 136.7282) (end 138.811 136.7282) (width 0.25) (layer F.Cu) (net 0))
 (segment (start 136.4488 136.271) (end 136.906 136.7282) (width 0.25) (layer F.Cu) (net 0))
 (segment (start 134.7088 136.271) (end 136.4488 136.271) (width 0.25) (layer F.Cu) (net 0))
 (segment (start 134.6898 136.29) (end 134.7088 136.271) (width 0.25) (layer F.Cu) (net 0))
 (segment (start 134.0398 135.0486) (end 134.0398 136.402) (width 0.25) (layer F.Cu) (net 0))
 (segment (start 140.9954 137.6426) (end 142.5448 139.192) (width 0.25) (layer F.Cu) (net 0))
 (segment (start 139.0904 137.6426) (end 140.9954 137.6426) (width 0.25) (layer F.Cu) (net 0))
 (segment (start 138.6332 137.1854) (end 139.0904 137.6426) (width 0.25) (layer F.Cu) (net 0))
 (segment (start 136.7282 137.1854) (end 138.6332 137.1854) (width 0.25) (layer F.Cu) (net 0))
 (segment (start 136.271 136.7282) (end 136.7282 137.1854) (width 0.25) (layer F.Cu) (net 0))
 (segment (start 134.366 136.7282) (end 136.271 136.7282) (width 0.25) (layer F.Cu) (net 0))
 (segment (start 134.0398 136.402) (end 134.366 136.7282) (width 0.25) (layer F.Cu) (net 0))
 (segment (start 133.3898 135.0486) (end 133.3898 136.387) (width 0.25) (layer F.Cu) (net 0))
 (segment (start 138.4554 137.6426) (end 140.0048 139.192) (width 0.25) (layer F.Cu) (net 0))
 (segment (start 136.5504 137.6426) (end 138.4554 137.6426) (width 0.25) (layer F.Cu) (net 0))
 (segment (start 136.0932 137.1854) (end 136.5504 137.6426) (width 0.25) (layer F.Cu) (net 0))
 (segment (start 134.1882 137.1854) (end 136.0932 137.1854) (width 0.25) (layer F.Cu) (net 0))
 (segment (start 133.3898 136.387) (end 134.1882 137.1854) (width 0.25) (layer F.Cu) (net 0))
 (segment (start 132.7398 135.0486) (end 132.7398 136.372) (width 0.25) (layer F.Cu) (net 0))
 (segment (start 135.9154 137.6426) (end 137.4648 139.192) (width 0.25) (layer F.Cu) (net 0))
 (segment (start 134.0104 137.6426) (end 135.9154 137.6426) (width 0.25) (layer F.Cu) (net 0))
 (segment (start 132.7398 136.372) (end 134.0104 137.6426) (width 0.25) (layer F.Cu) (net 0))
 (segment (start 130.1398 135.0486) (end 130.1398 136.357) (width 0.25) (layer F.Cu) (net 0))
 (segment (start 130.1398 136.357) (end 127.3048 139.192) (width 0.25) (layer F.Cu) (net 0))
 (segment (start 132.0898 135.0486) (end 132.0898 136.357) (width 0.25) (layer F.Cu) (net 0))
 (segment (start 132.0898 136.357) (end 134.9248 139.192) (width 0.25) (layer F.Cu) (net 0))
 (segment (start 130.7898 135.0486) (end 130.7898 138.247) (width 0.25) (layer F.Cu) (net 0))
 (segment (start 130.7898 138.247) (end 129.8448 139.192) (width 0.25) (layer F.Cu) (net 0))
 (segment (start 131.4398 135.0486) (end 131.4398 138.247) (width 0.25) (layer F.Cu) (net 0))
 (segment (start 131.4398 138.247) (end 132.3848 139.192) (width 0.25) (layer F.Cu) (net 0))
 (segment (start 128.8398 128.2986) (end 128.8398 126.9602) (width 0.25) (layer F.Cu) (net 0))
 (segment (start 123.7742 125.7046) (end 122.2248 124.1552) (width 0.25) (layer F.Cu) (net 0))
 (segment (start 125.6792 125.7046) (end 123.7742 125.7046) (width 0.25) (layer F.Cu) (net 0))
 (segment (start 126.1364 126.1618) (end 125.6792 125.7046) (width 0.25) (layer F.Cu) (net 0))
 (segment (start 128.0414 126.1618) (end 126.1364 126.1618) (width 0.25) (layer F.Cu) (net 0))
 (segment (start 128.8398 126.9602) (end 128.0414 126.1618) (width 0.25) (layer F.Cu) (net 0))
 (segment (start 129.4898 128.2986) (end 129.4898 126.9752) (width 0.25) (layer F.Cu) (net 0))
 (segment (start 126.3142 125.7046) (end 124.7648 124.1552) (width 0.25) (layer F.Cu) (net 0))
 (segment (start 128.2192 125.7046) (end 126.3142 125.7046) (width 0.25) (layer F.Cu) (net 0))
 (segment (start 129.4898 126.9752) (end 128.2192 125.7046) (width 0.25) (layer F.Cu) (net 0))
 (segment (start 130.1398 128.2986) (end 130.1398 126.9902) (width 0.25) (layer F.Cu) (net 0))
 (segment (start 130.1398 126.9902) (end 127.3048 124.1552) (width 0.25) (layer F.Cu) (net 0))
 (segment (start 130.7898 128.2986) (end 130.7898 125.1002) (width 0.25) (layer F.Cu) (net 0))
 (segment (start 130.7898 125.1002) (end 129.8448 124.1552) (width 0.25) (layer F.Cu) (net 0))
 (segment (start 134.6898 128.2986) (end 134.6898 127.0572) (width 0.25) (layer F.Cu) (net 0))
 (segment (start 143.5354 125.7046) (end 145.0848 124.1552) (width 0.25) (layer F.Cu) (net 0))
 (segment (start 141.6304 125.7046) (end 143.5354 125.7046) (width 0.25) (layer F.Cu) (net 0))
 (segment (start 141.1732 126.1618) (end 141.6304 125.7046) (width 0.25) (layer F.Cu) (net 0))
 (segment (start 139.2682 126.1618) (end 141.1732 126.1618) (width 0.25) (layer F.Cu) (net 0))
 (segment (start 138.811 126.619) (end 139.2682 126.1618) (width 0.25) (layer F.Cu) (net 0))
 (segment (start 136.906 126.619) (end 138.811 126.619) (width 0.25) (layer F.Cu) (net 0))
 (segment (start 136.4488 127.0762) (end 136.906 126.619) (width 0.25) (layer F.Cu) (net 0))
 (segment (start 134.7088 127.0762) (end 136.4488 127.0762) (width 0.25) (layer F.Cu) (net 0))
 (segment (start 134.6898 127.0572) (end 134.7088 127.0762) (width 0.25) (layer F.Cu) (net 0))
 (segment (start 134.0398 128.2986) (end 134.0398 126.9452) (width 0.25) (layer F.Cu) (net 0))
 (segment (start 140.9954 125.7046) (end 142.5448 124.1552) (width 0.25) (layer F.Cu) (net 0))
 (segment (start 139.0904 125.7046) (end 140.9954 125.7046) (width 0.25) (layer F.Cu) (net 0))
 (segment (start 138.6332 126.1618) (end 139.0904 125.7046) (width 0.25) (layer F.Cu) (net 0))
 (segment (start 136.7282 126.1618) (end 138.6332 126.1618) (width 0.25) (layer F.Cu) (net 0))
 (segment (start 136.271 126.619) (end 136.7282 126.1618) (width 0.25) (layer F.Cu) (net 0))
 (segment (start 134.366 126.619) (end 136.271 126.619) (width 0.25) (layer F.Cu) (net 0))
 (segment (start 134.0398 126.9452) (end 134.366 126.619) (width 0.25) (layer F.Cu) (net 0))
 (segment (start 133.3898 128.2986) (end 133.3898 126.9602) (width 0.25) (layer F.Cu) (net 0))
 (segment (start 138.4554 125.7046) (end 140.0048 124.1552) (width 0.25) (layer F.Cu) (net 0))
 (segment (start 136.5504 125.7046) (end 138.4554 125.7046) (width 0.25) (layer F.Cu) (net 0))
 (segment (start 136.0932 126.1618) (end 136.5504 125.7046) (width 0.25) (layer F.Cu) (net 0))
 (segment (start 134.1882 126.1618) (end 136.0932 126.1618) (width 0.25) (layer F.Cu) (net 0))
 (segment (start 133.3898 126.9602) (end 134.1882 126.1618) (width 0.25) (layer F.Cu) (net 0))
 (segment (start 132.7398 128.2986) (end 132.7398 126.9752) (width 0.25) (layer F.Cu) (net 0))
 (segment (start 135.9154 125.7046) (end 137.4648 124.1552) (width 0.25) (layer F.Cu) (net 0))
 (segment (start 134.0104 125.7046) (end 135.9154 125.7046) (width 0.25) (layer F.Cu) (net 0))
 (segment (start 132.7398 126.9752) (end 134.0104 125.7046) (width 0.25) (layer F.Cu) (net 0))
 (segment (start 132.0898 128.2986) (end 132.0898 126.9902) (width 0.25) (layer F.Cu) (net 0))
 (segment (start 132.0898 126.9902) (end 134.9248 124.1552) (width 0.25) (layer F.Cu) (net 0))
 (segment (start 131.4398 128.2986) (end 131.4398 125.1002) (width 0.25) (layer F.Cu) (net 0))
 (segment (start 131.4398 125.1002) (end 132.3848 124.1552) (width 0.25) (layer F.Cu) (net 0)))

